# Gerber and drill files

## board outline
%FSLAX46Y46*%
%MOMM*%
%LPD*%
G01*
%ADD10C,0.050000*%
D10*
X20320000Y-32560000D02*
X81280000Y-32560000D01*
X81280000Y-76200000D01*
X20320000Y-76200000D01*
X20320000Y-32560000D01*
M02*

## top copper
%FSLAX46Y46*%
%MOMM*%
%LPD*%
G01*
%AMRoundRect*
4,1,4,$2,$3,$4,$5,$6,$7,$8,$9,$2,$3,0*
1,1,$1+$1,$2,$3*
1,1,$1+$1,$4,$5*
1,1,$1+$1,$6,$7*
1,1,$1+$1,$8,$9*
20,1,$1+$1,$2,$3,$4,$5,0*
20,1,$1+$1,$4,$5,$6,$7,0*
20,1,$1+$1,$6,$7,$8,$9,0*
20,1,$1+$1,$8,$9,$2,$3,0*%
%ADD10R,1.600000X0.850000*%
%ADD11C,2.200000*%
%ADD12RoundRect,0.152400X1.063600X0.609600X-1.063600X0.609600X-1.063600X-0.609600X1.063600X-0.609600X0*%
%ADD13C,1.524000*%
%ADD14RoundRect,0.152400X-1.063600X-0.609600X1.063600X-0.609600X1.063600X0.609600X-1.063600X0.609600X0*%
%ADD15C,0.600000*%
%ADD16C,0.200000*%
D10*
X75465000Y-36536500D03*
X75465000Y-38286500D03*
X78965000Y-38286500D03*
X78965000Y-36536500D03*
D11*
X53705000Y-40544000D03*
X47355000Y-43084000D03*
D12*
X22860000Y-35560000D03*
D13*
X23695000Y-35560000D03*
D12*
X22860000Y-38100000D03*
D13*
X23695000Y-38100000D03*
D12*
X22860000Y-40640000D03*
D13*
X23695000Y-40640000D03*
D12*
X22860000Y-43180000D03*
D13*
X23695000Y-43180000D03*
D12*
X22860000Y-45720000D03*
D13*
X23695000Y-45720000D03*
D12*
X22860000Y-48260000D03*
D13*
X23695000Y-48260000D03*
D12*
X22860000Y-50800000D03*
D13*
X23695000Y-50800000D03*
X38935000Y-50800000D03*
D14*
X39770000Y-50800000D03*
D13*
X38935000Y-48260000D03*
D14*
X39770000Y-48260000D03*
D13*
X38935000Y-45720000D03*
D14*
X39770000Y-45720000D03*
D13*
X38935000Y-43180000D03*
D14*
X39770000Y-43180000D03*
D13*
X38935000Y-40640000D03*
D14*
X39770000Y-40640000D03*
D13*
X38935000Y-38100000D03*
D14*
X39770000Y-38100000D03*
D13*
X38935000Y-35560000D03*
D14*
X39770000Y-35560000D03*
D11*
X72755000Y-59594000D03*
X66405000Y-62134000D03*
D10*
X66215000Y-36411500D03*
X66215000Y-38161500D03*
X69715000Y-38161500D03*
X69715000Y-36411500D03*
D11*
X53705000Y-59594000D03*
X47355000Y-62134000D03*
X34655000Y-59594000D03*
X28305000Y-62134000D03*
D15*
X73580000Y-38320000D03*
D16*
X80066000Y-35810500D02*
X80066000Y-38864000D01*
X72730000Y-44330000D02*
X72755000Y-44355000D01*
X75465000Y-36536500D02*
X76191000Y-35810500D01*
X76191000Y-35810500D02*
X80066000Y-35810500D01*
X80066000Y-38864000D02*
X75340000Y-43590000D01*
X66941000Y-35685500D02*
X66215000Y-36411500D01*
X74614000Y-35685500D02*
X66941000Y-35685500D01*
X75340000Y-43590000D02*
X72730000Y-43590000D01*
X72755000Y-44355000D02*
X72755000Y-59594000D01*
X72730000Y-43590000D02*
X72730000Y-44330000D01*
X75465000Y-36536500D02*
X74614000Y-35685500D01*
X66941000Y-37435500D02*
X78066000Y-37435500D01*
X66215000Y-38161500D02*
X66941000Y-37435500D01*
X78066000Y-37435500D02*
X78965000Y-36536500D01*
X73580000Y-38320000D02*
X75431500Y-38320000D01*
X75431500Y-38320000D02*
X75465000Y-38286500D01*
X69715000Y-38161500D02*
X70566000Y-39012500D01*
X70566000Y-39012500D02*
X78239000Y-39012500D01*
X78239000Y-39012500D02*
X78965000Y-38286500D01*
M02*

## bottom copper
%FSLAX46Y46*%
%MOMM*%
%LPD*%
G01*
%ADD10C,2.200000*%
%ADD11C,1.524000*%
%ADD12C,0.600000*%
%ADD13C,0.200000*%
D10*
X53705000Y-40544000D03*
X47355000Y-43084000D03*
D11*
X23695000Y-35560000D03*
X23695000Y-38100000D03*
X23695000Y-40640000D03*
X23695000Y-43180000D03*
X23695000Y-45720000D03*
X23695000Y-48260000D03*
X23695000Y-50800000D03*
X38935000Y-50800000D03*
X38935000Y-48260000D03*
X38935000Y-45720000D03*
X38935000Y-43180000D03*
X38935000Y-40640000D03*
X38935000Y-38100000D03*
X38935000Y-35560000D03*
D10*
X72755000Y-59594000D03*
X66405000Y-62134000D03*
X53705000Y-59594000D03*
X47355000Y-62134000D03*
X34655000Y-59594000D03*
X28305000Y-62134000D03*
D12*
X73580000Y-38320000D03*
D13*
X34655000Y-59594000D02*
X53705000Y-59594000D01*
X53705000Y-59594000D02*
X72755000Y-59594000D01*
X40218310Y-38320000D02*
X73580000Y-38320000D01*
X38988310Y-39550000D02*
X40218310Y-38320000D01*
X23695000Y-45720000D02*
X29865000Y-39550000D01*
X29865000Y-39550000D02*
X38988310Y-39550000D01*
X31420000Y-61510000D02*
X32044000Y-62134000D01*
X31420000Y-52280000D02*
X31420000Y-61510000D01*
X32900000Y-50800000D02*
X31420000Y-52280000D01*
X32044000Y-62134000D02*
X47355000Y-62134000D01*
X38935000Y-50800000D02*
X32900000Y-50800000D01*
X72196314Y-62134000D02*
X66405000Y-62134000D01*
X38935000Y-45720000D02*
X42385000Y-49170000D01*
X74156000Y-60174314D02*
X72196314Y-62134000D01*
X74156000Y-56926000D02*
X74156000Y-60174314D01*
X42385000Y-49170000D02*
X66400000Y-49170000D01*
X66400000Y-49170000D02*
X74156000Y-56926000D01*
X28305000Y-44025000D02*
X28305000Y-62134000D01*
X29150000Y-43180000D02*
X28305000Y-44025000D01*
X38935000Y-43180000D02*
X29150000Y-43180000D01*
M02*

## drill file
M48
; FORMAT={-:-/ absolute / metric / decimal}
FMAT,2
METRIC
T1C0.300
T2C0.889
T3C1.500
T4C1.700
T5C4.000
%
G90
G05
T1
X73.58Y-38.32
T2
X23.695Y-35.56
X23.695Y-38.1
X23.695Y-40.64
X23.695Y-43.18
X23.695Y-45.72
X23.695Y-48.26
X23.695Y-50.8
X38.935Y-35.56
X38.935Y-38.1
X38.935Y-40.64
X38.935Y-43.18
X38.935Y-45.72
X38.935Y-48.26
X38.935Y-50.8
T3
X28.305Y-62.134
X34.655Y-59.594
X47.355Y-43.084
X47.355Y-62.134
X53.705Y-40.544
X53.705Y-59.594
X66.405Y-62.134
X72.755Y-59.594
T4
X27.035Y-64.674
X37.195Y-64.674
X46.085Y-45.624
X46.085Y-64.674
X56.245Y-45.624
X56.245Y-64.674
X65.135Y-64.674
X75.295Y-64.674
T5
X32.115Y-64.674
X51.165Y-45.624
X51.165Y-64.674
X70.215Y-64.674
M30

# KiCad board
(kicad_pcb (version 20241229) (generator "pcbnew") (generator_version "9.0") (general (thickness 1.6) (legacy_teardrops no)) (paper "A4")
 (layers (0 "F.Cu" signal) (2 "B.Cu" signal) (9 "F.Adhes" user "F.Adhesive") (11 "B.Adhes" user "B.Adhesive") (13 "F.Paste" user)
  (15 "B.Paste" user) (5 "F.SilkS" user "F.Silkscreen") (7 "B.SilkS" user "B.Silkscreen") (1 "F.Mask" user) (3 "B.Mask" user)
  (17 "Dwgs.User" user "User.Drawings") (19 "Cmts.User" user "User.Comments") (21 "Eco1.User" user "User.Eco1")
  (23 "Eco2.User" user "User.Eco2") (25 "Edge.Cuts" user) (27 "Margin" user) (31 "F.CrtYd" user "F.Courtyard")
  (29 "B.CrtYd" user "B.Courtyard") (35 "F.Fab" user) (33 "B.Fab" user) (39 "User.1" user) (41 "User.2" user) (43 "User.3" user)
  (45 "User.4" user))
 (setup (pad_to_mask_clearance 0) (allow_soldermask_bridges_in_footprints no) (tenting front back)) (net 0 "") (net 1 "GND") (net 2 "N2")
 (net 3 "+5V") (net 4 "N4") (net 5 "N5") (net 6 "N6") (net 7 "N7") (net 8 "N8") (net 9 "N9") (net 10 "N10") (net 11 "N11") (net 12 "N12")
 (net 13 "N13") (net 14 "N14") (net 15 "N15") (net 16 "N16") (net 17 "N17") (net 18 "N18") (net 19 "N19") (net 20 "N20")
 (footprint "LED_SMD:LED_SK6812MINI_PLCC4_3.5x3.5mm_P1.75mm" (layer "F.Cu") (at 77.215 37.4115)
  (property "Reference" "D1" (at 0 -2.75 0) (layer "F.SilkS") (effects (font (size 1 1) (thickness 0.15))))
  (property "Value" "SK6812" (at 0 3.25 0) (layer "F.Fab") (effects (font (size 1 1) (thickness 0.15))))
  (pad "1" smd rect (at -1.75 -0.875) (size 1.6 0.85) (layers "F.Cu" "F.Mask" "F.Paste") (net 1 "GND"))
  (pad "2" smd rect (at -1.75 0.875) (size 1.6 0.85) (layers "F.Cu" "F.Mask" "F.Paste") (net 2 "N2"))
  (pad "3" smd rect (at 1.75 0.875) (size 1.6 0.85) (layers "F.Cu" "F.Mask" "F.Paste") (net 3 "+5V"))
  (pad "4" smd rect (at 1.75 -0.875) (size 1.6 0.85) (layers "F.Cu" "F.Mask" "F.Paste") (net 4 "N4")))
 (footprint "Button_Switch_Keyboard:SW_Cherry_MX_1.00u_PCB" (layer "F.Cu") (at 53.705 40.544)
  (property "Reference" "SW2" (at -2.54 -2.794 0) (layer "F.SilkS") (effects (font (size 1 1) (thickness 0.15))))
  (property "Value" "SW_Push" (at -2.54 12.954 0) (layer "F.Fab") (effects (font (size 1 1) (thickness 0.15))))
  (pad "" np_thru_hole circle (at -7.62 5.08) (size 1.7 1.7) (drill 1.7) (layers "*.Cu" "*.Mask"))
  (pad "" np_thru_hole circle (at -2.54 5.08) (size 4 4) (drill 4) (layers "*.Cu" "*.Mask"))
  (pad "" np_thru_hole circle (at 2.54 5.08) (size 1.7 1.7) (drill 1.7) (layers "*.Cu" "*.Mask"))
  (pad "1" thru_hole circle (at 0 0) (size 2.2 2.2) (drill 1.5) (layers "*.Cu" "*.Mask") (remove_unused_layers no) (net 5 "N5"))
  (pad "2" thru_hole circle (at -6.35 2.54) (size 2.2 2.2) (drill 1.5) (layers "*.Cu" "*.Mask") (remove_unused_layers no) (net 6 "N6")))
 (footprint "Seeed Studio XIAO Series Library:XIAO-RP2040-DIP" (layer "F.Cu") (at 31.315 43.18)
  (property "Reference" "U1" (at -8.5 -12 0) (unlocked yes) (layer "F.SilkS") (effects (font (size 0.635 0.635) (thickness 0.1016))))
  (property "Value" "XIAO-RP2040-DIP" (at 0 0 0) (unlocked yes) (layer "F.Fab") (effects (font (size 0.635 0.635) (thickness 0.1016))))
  (pad "1" smd roundrect (at -8.455 -7.62 180) (size 2.432 1.524) (layers "F.Cu" "F.Mask") (roundrect_rratio 0.1) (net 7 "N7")
   (thermal_bridge_angle 45))
  (pad "1" thru_hole circle (at -7.62 -7.62 180) (size 1.524 1.524) (drill 0.889) (layers "*.Cu" "*.Mask") (remove_unused_layers no)
   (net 7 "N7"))
  (pad "2" smd roundrect (at -8.455 -5.08 180) (size 2.432 1.524) (layers "F.Cu" "F.Mask") (roundrect_rratio 0.1) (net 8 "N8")
   (thermal_bridge_angle 45))
  (pad "2" thru_hole circle (at -7.62 -5.08 180) (size 1.524 1.524) (drill 0.889) (layers "*.Cu" "*.Mask") (remove_unused_layers no)
   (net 8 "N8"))
  (pad "3" smd roundrect (at -8.455 -2.54 180) (size 2.432 1.524) (layers "F.Cu" "F.Mask") (roundrect_rratio 0.1) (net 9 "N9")
   (thermal_bridge_angle 45))
  (pad "3" thru_hole circle (at -7.62 -2.54 180) (size 1.524 1.524) (drill 0.889) (layers "*.Cu" "*.Mask") (remove_unused_layers no)
   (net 9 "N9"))
  (pad "4" smd roundrect (at -8.455 0 180) (size 2.432 1.524) (layers "F.Cu" "F.Mask") (roundrect_rratio 0.1) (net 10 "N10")
   (thermal_bridge_angle 45))
  (pad "4" thru_hole circle (at -7.62 0 180) (size 1.524 1.524) (drill 0.889) (layers "*.Cu" "*.Mask") (remove_unused_layers no)
   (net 10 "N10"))
  (pad "5" smd roundrect (at -8.455 2.54 180) (size 2.432 1.524) (layers "F.Cu" "F.Mask") (roundrect_rratio 0.1) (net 2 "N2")
   (thermal_bridge_angle 45))
  (pad "5" thru_hole circle (at -7.62 2.54 180) (size 1.524 1.524) (drill 0.889) (layers "*.Cu" "*.Mask") (remove_unused_layers no)
   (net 2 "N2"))
  (pad "6" smd roundrect (at -8.455 5.08 180) (size 2.432 1.524) (layers "F.Cu" "F.Mask") (roundrect_rratio 0.1) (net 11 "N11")
   (thermal_bridge_angle 45))
  (pad "6" thru_hole circle (at -7.62 5.08 180) (size 1.524 1.524) (drill 0.889) (layers "*.Cu" "*.Mask") (remove_unused_layers no)
   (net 11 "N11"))
  (pad "7" smd roundrect (at -8.455 7.62 180) (size 2.432 1.524) (layers "F.Cu" "F.Mask") (roundrect_rratio 0.1) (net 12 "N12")
   (thermal_bridge_angle 45))
  (pad "7" thru_hole circle (at -7.62 7.62 180) (size 1.524 1.524) (drill 0.889) (layers "*.Cu" "*.Mask") (remove_unused_layers no)
   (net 12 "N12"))
  (pad "8" thru_hole circle (at 7.62 7.62) (size 1.524 1.524) (drill 0.889) (layers "*.Cu" "*.Mask") (remove_unused_layers no)
   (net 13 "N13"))
  (pad "8" smd roundrect (at 8.455 7.62) (size 2.432 1.524) (layers "F.Cu" "F.Mask") (roundrect_rratio 0.1) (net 13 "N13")
   (thermal_bridge_angle 45))
  (pad "9" thru_hole circle (at 7.62 5.08) (size 1.524 1.524) (drill 0.889) (layers "*.Cu" "*.Mask") (remove_unused_layers no)
   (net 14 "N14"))
  (pad "9" smd roundrect (at 8.455 5.08) (size 2.432 1.524) (layers "F.Cu" "F.Mask") (roundrect_rratio 0.1) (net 14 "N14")
   (thermal_bridge_angle 45))
  (pad "10" thru_hole circle (at 7.62 2.54) (size 1.524 1.524) (drill 0.889) (layers "*.Cu" "*.Mask") (remove_unused_layers no)
   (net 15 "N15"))
  (pad "10" smd roundrect (at 8.455 2.54) (size 2.432 1.524) (layers "F.Cu" "F.Mask") (roundrect_rratio 0.1) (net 15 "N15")
   (thermal_bridge_angle 45))
  (pad "11" thru_hole circle (at 7.62 0) (size 1.524 1.524) (drill 0.889) (layers "*.Cu" "*.Mask") (remove_unused_layers no) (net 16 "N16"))
  (pad "11" smd roundrect (at 8.455 0) (size 2.432 1.524) (layers "F.Cu" "F.Mask") (roundrect_rratio 0.1) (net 16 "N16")
   (thermal_bridge_angle 45))
  (pad "12" thru_hole circle (at 7.62 -2.54) (size 1.524 1.524) (drill 0.889) (layers "*.Cu" "*.Mask") (remove_unused_layers no)
   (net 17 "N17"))
  (pad "12" smd roundrect (at 8.455 -2.54) (size 2.432 1.524) (layers "F.Cu" "F.Mask") (roundrect_rratio 0.1) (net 17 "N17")
   (thermal_bridge_angle 45))
  (pad "13" thru_hole circle (at 7.62 -5.08) (size 1.524 1.524) (drill 0.889) (layers "*.Cu" "*.Mask") (remove_unused_layers no)
   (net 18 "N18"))
  (pad "13" smd roundrect (at 8.455 -5.08) (size 2.432 1.524) (layers "F.Cu" "F.Mask") (roundrect_rratio 0.1) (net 18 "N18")
   (thermal_bridge_angle 45))
  (pad "14" thru_hole circle (at 7.62 -7.62) (size 1.524 1.524) (drill 0.889) (layers "*.Cu" "*.Mask") (remove_unused_layers no)
   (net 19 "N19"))
  (pad "14" smd roundrect (at 8.455 -7.62) (size 2.432 1.524) (layers "F.Cu" "F.Mask") (roundrect_rratio 0.1) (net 19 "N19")
   (thermal_bridge_angle 45)))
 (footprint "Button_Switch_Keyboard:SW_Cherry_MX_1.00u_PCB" (layer "F.Cu") (at 72.755 59.594)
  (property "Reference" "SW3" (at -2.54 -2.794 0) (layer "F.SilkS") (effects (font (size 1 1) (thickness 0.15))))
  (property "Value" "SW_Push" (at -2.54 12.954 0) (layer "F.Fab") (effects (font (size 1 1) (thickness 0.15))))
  (pad "" np_thru_hole circle (at -7.62 5.08) (size 1.7 1.7) (drill 1.7) (layers "*.Cu" "*.Mask"))
  (pad "" np_thru_hole circle (at -2.54 5.08) (size 4 4) (drill 4) (layers "*.Cu" "*.Mask"))
  (pad "" np_thru_hole circle (at 2.54 5.08) (size 1.7 1.7) (drill 1.7) (layers "*.Cu" "*.Mask"))
  (pad "1" thru_hole circle (at 0 0) (size 2.2 2.2) (drill 1.5) (layers "*.Cu" "*.Mask") (remove_unused_layers no) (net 1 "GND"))
  (pad "2" thru_hole circle (at -6.35 2.54) (size 2.2 2.2) (drill 1.5) (layers "*.Cu" "*.Mask") (remove_unused_layers no) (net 15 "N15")))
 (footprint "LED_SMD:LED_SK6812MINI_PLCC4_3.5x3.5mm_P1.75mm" (layer "F.Cu") (at 67.965 37.2865)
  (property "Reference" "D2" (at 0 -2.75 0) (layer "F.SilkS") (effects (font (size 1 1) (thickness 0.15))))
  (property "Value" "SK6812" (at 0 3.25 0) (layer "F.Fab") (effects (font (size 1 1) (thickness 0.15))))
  (pad "1" smd rect (at -1.75 -0.875) (size 1.6 0.85) (layers "F.Cu" "F.Mask" "F.Paste") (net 1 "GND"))
  (pad "2" smd rect (at -1.75 0.875) (size 1.6 0.85) (layers "F.Cu" "F.Mask" "F.Paste") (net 4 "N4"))
  (pad "3" smd rect (at 1.75 0.875) (size 1.6 0.85) (layers "F.Cu" "F.Mask" "F.Paste") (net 3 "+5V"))
  (pad "4" smd rect (at 1.75 -0.875) (size 1.6 0.85) (layers "F.Cu" "F.Mask" "F.Paste") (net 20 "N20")))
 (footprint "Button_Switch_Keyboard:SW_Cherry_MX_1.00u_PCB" (layer "F.Cu") (at 53.705 59.594)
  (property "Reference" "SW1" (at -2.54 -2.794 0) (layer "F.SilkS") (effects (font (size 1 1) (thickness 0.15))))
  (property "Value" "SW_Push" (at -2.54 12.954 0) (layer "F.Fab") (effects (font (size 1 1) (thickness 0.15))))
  (pad "" np_thru_hole circle (at -7.62 5.08) (size 1.7 1.7) (drill 1.7) (layers "*.Cu" "*.Mask"))
  (pad "" np_thru_hole circle (at -2.54 5.08) (size 4 4) (drill 4) (layers "*.Cu" "*.Mask"))
  (pad "" np_thru_hole circle (at 2.54 5.08) (size 1.7 1.7) (drill 1.7) (layers "*.Cu" "*.Mask"))
  (pad "1" thru_hole circle (at 0 0) (size 2.2 2.2) (drill 1.5) (layers "*.Cu" "*.Mask") (remove_unused_layers no) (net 1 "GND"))
  (pad "2" thru_hole circle (at -6.35 2.54) (size 2.2 2.2) (drill 1.5) (layers "*.Cu" "*.Mask") (remove_unused_layers no) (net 13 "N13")))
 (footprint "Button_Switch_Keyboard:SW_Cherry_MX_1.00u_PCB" (layer "F.Cu") (at 34.655 59.594)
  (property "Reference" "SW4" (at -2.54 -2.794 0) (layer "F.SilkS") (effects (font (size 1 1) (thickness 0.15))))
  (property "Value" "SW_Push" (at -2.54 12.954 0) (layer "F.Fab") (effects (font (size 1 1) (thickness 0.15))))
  (pad "" np_thru_hole circle (at -7.62 5.08) (size 1.7 1.7) (drill 1.7) (layers "*.Cu" "*.Mask"))
  (pad "" np_thru_hole circle (at -2.54 5.08) (size 4 4) (drill 4) (layers "*.Cu" "*.Mask"))
  (pad "" np_thru_hole circle (at 2.54 5.08) (size 1.7 1.7) (drill 1.7) (layers "*.Cu" "*.Mask"))
  (pad "1" thru_hole circle (at 0 0) (size 2.2 2.2) (drill 1.5) (layers "*.Cu" "*.Mask") (remove_unused_layers no) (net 1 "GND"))
  (pad "2" thru_hole circle (at -6.35 2.54) (size 2.2 2.2) (drill 1.5) (layers "*.Cu" "*.Mask") (remove_unused_layers no) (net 16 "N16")))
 (gr_rect (start 20.32 32.56) (end 81.28 76.2) (stroke (width 0.05) (type default)) (fill no) (layer "Edge.Cuts"))
 (segment (start 80.066 35.8105) (end 80.066 38.864) (width 0.2) (layer "F.Cu") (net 1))
 (segment (start 72.73 44.33) (end 72.755 44.355) (width 0.2) (layer "F.Cu") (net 1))
 (segment (start 75.465 36.5365) (end 76.191 35.8105) (width 0.2) (layer "F.Cu") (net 1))
 (segment (start 76.191 35.8105) (end 80.066 35.8105) (width 0.2) (layer "F.Cu") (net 1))
 (segment (start 80.066 38.864) (end 75.34 43.59) (width 0.2) (layer "F.Cu") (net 1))
 (segment (start 66.941 35.6855) (end 66.215 36.4115) (width 0.2) (layer "F.Cu") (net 1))
 (segment (start 74.614 35.6855) (end 66.941 35.6855) (width 0.2) (layer "F.Cu") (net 1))
 (segment (start 75.34 43.59) (end 72.73 43.59) (width 0.2) (layer "F.Cu") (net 1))
 (segment (start 72.755 44.355) (end 72.755 59.594) (width 0.2) (layer "F.Cu") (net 1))
 (segment (start 72.73 43.59) (end 72.73 44.33) (width 0.2) (layer "F.Cu") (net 1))
 (segment (start 75.465 36.5365) (end 74.614 35.6855) (width 0.2) (layer "F.Cu") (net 1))
 (segment (start 34.655 59.594) (end 53.705 59.594) (width 0.2) (layer "B.Cu") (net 1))
 (segment (start 53.705 59.594) (end 72.755 59.594) (width 0.2) (layer "B.Cu") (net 1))
 (segment (start 66.941 37.4355) (end 78.066 37.4355) (width 0.2) (layer "F.Cu") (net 4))
 (segment (start 66.215 38.1615) (end 66.941 37.4355) (width 0.2) (layer "F.Cu") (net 4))
 (segment (start 78.066 37.4355) (end 78.965 36.5365) (width 0.2) (layer "F.Cu") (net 4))
 (segment (start 73.58 38.32) (end 75.4315 38.32) (width 0.2) (layer "F.Cu") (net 2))
 (segment (start 75.4315 38.32) (end 75.465 38.2865) (width 0.2) (layer "F.Cu") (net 2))
 (via (at 73.58 38.32) (size 0.6) (drill 0.3) (layers "F.Cu" "B.Cu") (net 2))
 (segment (start 40.21831 38.32) (end 73.58 38.32) (width 0.2) (layer "B.Cu") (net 2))
 (segment (start 38.98831 39.55) (end 40.21831 38.32) (width 0.2) (layer "B.Cu") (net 2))
 (segment (start 23.695 45.72) (end 29.865 39.55) (width 0.2) (layer "B.Cu") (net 2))
 (segment (start 29.865 39.55) (end 38.98831 39.55) (width 0.2) (layer "B.Cu") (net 2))
 (segment (start 69.715 38.1615) (end 70.566 39.0125) (width 0.2) (layer "F.Cu") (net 3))
 (segment (start 70.566 39.0125) (end 78.239 39.0125) (width 0.2) (layer "F.Cu") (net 3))
 (segment (start 78.239 39.0125) (end 78.965 38.2865) (width 0.2) (layer "F.Cu") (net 3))
 (segment (start 31.42 61.51) (end 32.044 62.134) (width 0.2) (layer "B.Cu") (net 13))
 (segment (start 31.42 52.28) (end 31.42 61.51) (width 0.2) (layer "B.Cu") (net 13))
 (segment (start 32.9 50.8) (end 31.42 52.28) (width 0.2) (layer "B.Cu") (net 13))
 (segment (start 32.044 62.134) (end 47.355 62.134) (width 0.2) (layer "B.Cu") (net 13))
 (segment (start 38.935 50.8) (end 32.9 50.8) (width 0.2) (layer "B.Cu") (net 13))
 (segment (start 72.196314 62.134) (end 66.405 62.134) (width 0.2) (layer "B.Cu") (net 15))
 (segment (start 38.935 45.72) (end 42.385 49.17) (width 0.2) (layer "B.Cu") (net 15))
 (segment (start 74.156 60.174314) (end 72.196314 62.134) (width 0.2) (layer "B.Cu") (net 15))
 (segment (start 74.156 56.926) (end 74.156 60.174314) (width 0.2) (layer "B.Cu") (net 15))
 (segment (start 42.385 49.17) (end 66.4 49.17) (width 0.2) (layer "B.Cu") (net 15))
 (segment (start 66.4 49.17) (end 74.156 56.926) (width 0.2) (layer "B.Cu") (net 15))
 (segment (start 28.305 44.025) (end 28.305 62.134) (width 0.2) (layer "B.Cu") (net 16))
 (segment (start 29.15 43.18) (end 28.305 44.025) (width 0.2) (layer "B.Cu") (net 16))
 (segment (start 38.935 43.18) (end 29.15 43.18) (width 0.2) (layer "B.Cu") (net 16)))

